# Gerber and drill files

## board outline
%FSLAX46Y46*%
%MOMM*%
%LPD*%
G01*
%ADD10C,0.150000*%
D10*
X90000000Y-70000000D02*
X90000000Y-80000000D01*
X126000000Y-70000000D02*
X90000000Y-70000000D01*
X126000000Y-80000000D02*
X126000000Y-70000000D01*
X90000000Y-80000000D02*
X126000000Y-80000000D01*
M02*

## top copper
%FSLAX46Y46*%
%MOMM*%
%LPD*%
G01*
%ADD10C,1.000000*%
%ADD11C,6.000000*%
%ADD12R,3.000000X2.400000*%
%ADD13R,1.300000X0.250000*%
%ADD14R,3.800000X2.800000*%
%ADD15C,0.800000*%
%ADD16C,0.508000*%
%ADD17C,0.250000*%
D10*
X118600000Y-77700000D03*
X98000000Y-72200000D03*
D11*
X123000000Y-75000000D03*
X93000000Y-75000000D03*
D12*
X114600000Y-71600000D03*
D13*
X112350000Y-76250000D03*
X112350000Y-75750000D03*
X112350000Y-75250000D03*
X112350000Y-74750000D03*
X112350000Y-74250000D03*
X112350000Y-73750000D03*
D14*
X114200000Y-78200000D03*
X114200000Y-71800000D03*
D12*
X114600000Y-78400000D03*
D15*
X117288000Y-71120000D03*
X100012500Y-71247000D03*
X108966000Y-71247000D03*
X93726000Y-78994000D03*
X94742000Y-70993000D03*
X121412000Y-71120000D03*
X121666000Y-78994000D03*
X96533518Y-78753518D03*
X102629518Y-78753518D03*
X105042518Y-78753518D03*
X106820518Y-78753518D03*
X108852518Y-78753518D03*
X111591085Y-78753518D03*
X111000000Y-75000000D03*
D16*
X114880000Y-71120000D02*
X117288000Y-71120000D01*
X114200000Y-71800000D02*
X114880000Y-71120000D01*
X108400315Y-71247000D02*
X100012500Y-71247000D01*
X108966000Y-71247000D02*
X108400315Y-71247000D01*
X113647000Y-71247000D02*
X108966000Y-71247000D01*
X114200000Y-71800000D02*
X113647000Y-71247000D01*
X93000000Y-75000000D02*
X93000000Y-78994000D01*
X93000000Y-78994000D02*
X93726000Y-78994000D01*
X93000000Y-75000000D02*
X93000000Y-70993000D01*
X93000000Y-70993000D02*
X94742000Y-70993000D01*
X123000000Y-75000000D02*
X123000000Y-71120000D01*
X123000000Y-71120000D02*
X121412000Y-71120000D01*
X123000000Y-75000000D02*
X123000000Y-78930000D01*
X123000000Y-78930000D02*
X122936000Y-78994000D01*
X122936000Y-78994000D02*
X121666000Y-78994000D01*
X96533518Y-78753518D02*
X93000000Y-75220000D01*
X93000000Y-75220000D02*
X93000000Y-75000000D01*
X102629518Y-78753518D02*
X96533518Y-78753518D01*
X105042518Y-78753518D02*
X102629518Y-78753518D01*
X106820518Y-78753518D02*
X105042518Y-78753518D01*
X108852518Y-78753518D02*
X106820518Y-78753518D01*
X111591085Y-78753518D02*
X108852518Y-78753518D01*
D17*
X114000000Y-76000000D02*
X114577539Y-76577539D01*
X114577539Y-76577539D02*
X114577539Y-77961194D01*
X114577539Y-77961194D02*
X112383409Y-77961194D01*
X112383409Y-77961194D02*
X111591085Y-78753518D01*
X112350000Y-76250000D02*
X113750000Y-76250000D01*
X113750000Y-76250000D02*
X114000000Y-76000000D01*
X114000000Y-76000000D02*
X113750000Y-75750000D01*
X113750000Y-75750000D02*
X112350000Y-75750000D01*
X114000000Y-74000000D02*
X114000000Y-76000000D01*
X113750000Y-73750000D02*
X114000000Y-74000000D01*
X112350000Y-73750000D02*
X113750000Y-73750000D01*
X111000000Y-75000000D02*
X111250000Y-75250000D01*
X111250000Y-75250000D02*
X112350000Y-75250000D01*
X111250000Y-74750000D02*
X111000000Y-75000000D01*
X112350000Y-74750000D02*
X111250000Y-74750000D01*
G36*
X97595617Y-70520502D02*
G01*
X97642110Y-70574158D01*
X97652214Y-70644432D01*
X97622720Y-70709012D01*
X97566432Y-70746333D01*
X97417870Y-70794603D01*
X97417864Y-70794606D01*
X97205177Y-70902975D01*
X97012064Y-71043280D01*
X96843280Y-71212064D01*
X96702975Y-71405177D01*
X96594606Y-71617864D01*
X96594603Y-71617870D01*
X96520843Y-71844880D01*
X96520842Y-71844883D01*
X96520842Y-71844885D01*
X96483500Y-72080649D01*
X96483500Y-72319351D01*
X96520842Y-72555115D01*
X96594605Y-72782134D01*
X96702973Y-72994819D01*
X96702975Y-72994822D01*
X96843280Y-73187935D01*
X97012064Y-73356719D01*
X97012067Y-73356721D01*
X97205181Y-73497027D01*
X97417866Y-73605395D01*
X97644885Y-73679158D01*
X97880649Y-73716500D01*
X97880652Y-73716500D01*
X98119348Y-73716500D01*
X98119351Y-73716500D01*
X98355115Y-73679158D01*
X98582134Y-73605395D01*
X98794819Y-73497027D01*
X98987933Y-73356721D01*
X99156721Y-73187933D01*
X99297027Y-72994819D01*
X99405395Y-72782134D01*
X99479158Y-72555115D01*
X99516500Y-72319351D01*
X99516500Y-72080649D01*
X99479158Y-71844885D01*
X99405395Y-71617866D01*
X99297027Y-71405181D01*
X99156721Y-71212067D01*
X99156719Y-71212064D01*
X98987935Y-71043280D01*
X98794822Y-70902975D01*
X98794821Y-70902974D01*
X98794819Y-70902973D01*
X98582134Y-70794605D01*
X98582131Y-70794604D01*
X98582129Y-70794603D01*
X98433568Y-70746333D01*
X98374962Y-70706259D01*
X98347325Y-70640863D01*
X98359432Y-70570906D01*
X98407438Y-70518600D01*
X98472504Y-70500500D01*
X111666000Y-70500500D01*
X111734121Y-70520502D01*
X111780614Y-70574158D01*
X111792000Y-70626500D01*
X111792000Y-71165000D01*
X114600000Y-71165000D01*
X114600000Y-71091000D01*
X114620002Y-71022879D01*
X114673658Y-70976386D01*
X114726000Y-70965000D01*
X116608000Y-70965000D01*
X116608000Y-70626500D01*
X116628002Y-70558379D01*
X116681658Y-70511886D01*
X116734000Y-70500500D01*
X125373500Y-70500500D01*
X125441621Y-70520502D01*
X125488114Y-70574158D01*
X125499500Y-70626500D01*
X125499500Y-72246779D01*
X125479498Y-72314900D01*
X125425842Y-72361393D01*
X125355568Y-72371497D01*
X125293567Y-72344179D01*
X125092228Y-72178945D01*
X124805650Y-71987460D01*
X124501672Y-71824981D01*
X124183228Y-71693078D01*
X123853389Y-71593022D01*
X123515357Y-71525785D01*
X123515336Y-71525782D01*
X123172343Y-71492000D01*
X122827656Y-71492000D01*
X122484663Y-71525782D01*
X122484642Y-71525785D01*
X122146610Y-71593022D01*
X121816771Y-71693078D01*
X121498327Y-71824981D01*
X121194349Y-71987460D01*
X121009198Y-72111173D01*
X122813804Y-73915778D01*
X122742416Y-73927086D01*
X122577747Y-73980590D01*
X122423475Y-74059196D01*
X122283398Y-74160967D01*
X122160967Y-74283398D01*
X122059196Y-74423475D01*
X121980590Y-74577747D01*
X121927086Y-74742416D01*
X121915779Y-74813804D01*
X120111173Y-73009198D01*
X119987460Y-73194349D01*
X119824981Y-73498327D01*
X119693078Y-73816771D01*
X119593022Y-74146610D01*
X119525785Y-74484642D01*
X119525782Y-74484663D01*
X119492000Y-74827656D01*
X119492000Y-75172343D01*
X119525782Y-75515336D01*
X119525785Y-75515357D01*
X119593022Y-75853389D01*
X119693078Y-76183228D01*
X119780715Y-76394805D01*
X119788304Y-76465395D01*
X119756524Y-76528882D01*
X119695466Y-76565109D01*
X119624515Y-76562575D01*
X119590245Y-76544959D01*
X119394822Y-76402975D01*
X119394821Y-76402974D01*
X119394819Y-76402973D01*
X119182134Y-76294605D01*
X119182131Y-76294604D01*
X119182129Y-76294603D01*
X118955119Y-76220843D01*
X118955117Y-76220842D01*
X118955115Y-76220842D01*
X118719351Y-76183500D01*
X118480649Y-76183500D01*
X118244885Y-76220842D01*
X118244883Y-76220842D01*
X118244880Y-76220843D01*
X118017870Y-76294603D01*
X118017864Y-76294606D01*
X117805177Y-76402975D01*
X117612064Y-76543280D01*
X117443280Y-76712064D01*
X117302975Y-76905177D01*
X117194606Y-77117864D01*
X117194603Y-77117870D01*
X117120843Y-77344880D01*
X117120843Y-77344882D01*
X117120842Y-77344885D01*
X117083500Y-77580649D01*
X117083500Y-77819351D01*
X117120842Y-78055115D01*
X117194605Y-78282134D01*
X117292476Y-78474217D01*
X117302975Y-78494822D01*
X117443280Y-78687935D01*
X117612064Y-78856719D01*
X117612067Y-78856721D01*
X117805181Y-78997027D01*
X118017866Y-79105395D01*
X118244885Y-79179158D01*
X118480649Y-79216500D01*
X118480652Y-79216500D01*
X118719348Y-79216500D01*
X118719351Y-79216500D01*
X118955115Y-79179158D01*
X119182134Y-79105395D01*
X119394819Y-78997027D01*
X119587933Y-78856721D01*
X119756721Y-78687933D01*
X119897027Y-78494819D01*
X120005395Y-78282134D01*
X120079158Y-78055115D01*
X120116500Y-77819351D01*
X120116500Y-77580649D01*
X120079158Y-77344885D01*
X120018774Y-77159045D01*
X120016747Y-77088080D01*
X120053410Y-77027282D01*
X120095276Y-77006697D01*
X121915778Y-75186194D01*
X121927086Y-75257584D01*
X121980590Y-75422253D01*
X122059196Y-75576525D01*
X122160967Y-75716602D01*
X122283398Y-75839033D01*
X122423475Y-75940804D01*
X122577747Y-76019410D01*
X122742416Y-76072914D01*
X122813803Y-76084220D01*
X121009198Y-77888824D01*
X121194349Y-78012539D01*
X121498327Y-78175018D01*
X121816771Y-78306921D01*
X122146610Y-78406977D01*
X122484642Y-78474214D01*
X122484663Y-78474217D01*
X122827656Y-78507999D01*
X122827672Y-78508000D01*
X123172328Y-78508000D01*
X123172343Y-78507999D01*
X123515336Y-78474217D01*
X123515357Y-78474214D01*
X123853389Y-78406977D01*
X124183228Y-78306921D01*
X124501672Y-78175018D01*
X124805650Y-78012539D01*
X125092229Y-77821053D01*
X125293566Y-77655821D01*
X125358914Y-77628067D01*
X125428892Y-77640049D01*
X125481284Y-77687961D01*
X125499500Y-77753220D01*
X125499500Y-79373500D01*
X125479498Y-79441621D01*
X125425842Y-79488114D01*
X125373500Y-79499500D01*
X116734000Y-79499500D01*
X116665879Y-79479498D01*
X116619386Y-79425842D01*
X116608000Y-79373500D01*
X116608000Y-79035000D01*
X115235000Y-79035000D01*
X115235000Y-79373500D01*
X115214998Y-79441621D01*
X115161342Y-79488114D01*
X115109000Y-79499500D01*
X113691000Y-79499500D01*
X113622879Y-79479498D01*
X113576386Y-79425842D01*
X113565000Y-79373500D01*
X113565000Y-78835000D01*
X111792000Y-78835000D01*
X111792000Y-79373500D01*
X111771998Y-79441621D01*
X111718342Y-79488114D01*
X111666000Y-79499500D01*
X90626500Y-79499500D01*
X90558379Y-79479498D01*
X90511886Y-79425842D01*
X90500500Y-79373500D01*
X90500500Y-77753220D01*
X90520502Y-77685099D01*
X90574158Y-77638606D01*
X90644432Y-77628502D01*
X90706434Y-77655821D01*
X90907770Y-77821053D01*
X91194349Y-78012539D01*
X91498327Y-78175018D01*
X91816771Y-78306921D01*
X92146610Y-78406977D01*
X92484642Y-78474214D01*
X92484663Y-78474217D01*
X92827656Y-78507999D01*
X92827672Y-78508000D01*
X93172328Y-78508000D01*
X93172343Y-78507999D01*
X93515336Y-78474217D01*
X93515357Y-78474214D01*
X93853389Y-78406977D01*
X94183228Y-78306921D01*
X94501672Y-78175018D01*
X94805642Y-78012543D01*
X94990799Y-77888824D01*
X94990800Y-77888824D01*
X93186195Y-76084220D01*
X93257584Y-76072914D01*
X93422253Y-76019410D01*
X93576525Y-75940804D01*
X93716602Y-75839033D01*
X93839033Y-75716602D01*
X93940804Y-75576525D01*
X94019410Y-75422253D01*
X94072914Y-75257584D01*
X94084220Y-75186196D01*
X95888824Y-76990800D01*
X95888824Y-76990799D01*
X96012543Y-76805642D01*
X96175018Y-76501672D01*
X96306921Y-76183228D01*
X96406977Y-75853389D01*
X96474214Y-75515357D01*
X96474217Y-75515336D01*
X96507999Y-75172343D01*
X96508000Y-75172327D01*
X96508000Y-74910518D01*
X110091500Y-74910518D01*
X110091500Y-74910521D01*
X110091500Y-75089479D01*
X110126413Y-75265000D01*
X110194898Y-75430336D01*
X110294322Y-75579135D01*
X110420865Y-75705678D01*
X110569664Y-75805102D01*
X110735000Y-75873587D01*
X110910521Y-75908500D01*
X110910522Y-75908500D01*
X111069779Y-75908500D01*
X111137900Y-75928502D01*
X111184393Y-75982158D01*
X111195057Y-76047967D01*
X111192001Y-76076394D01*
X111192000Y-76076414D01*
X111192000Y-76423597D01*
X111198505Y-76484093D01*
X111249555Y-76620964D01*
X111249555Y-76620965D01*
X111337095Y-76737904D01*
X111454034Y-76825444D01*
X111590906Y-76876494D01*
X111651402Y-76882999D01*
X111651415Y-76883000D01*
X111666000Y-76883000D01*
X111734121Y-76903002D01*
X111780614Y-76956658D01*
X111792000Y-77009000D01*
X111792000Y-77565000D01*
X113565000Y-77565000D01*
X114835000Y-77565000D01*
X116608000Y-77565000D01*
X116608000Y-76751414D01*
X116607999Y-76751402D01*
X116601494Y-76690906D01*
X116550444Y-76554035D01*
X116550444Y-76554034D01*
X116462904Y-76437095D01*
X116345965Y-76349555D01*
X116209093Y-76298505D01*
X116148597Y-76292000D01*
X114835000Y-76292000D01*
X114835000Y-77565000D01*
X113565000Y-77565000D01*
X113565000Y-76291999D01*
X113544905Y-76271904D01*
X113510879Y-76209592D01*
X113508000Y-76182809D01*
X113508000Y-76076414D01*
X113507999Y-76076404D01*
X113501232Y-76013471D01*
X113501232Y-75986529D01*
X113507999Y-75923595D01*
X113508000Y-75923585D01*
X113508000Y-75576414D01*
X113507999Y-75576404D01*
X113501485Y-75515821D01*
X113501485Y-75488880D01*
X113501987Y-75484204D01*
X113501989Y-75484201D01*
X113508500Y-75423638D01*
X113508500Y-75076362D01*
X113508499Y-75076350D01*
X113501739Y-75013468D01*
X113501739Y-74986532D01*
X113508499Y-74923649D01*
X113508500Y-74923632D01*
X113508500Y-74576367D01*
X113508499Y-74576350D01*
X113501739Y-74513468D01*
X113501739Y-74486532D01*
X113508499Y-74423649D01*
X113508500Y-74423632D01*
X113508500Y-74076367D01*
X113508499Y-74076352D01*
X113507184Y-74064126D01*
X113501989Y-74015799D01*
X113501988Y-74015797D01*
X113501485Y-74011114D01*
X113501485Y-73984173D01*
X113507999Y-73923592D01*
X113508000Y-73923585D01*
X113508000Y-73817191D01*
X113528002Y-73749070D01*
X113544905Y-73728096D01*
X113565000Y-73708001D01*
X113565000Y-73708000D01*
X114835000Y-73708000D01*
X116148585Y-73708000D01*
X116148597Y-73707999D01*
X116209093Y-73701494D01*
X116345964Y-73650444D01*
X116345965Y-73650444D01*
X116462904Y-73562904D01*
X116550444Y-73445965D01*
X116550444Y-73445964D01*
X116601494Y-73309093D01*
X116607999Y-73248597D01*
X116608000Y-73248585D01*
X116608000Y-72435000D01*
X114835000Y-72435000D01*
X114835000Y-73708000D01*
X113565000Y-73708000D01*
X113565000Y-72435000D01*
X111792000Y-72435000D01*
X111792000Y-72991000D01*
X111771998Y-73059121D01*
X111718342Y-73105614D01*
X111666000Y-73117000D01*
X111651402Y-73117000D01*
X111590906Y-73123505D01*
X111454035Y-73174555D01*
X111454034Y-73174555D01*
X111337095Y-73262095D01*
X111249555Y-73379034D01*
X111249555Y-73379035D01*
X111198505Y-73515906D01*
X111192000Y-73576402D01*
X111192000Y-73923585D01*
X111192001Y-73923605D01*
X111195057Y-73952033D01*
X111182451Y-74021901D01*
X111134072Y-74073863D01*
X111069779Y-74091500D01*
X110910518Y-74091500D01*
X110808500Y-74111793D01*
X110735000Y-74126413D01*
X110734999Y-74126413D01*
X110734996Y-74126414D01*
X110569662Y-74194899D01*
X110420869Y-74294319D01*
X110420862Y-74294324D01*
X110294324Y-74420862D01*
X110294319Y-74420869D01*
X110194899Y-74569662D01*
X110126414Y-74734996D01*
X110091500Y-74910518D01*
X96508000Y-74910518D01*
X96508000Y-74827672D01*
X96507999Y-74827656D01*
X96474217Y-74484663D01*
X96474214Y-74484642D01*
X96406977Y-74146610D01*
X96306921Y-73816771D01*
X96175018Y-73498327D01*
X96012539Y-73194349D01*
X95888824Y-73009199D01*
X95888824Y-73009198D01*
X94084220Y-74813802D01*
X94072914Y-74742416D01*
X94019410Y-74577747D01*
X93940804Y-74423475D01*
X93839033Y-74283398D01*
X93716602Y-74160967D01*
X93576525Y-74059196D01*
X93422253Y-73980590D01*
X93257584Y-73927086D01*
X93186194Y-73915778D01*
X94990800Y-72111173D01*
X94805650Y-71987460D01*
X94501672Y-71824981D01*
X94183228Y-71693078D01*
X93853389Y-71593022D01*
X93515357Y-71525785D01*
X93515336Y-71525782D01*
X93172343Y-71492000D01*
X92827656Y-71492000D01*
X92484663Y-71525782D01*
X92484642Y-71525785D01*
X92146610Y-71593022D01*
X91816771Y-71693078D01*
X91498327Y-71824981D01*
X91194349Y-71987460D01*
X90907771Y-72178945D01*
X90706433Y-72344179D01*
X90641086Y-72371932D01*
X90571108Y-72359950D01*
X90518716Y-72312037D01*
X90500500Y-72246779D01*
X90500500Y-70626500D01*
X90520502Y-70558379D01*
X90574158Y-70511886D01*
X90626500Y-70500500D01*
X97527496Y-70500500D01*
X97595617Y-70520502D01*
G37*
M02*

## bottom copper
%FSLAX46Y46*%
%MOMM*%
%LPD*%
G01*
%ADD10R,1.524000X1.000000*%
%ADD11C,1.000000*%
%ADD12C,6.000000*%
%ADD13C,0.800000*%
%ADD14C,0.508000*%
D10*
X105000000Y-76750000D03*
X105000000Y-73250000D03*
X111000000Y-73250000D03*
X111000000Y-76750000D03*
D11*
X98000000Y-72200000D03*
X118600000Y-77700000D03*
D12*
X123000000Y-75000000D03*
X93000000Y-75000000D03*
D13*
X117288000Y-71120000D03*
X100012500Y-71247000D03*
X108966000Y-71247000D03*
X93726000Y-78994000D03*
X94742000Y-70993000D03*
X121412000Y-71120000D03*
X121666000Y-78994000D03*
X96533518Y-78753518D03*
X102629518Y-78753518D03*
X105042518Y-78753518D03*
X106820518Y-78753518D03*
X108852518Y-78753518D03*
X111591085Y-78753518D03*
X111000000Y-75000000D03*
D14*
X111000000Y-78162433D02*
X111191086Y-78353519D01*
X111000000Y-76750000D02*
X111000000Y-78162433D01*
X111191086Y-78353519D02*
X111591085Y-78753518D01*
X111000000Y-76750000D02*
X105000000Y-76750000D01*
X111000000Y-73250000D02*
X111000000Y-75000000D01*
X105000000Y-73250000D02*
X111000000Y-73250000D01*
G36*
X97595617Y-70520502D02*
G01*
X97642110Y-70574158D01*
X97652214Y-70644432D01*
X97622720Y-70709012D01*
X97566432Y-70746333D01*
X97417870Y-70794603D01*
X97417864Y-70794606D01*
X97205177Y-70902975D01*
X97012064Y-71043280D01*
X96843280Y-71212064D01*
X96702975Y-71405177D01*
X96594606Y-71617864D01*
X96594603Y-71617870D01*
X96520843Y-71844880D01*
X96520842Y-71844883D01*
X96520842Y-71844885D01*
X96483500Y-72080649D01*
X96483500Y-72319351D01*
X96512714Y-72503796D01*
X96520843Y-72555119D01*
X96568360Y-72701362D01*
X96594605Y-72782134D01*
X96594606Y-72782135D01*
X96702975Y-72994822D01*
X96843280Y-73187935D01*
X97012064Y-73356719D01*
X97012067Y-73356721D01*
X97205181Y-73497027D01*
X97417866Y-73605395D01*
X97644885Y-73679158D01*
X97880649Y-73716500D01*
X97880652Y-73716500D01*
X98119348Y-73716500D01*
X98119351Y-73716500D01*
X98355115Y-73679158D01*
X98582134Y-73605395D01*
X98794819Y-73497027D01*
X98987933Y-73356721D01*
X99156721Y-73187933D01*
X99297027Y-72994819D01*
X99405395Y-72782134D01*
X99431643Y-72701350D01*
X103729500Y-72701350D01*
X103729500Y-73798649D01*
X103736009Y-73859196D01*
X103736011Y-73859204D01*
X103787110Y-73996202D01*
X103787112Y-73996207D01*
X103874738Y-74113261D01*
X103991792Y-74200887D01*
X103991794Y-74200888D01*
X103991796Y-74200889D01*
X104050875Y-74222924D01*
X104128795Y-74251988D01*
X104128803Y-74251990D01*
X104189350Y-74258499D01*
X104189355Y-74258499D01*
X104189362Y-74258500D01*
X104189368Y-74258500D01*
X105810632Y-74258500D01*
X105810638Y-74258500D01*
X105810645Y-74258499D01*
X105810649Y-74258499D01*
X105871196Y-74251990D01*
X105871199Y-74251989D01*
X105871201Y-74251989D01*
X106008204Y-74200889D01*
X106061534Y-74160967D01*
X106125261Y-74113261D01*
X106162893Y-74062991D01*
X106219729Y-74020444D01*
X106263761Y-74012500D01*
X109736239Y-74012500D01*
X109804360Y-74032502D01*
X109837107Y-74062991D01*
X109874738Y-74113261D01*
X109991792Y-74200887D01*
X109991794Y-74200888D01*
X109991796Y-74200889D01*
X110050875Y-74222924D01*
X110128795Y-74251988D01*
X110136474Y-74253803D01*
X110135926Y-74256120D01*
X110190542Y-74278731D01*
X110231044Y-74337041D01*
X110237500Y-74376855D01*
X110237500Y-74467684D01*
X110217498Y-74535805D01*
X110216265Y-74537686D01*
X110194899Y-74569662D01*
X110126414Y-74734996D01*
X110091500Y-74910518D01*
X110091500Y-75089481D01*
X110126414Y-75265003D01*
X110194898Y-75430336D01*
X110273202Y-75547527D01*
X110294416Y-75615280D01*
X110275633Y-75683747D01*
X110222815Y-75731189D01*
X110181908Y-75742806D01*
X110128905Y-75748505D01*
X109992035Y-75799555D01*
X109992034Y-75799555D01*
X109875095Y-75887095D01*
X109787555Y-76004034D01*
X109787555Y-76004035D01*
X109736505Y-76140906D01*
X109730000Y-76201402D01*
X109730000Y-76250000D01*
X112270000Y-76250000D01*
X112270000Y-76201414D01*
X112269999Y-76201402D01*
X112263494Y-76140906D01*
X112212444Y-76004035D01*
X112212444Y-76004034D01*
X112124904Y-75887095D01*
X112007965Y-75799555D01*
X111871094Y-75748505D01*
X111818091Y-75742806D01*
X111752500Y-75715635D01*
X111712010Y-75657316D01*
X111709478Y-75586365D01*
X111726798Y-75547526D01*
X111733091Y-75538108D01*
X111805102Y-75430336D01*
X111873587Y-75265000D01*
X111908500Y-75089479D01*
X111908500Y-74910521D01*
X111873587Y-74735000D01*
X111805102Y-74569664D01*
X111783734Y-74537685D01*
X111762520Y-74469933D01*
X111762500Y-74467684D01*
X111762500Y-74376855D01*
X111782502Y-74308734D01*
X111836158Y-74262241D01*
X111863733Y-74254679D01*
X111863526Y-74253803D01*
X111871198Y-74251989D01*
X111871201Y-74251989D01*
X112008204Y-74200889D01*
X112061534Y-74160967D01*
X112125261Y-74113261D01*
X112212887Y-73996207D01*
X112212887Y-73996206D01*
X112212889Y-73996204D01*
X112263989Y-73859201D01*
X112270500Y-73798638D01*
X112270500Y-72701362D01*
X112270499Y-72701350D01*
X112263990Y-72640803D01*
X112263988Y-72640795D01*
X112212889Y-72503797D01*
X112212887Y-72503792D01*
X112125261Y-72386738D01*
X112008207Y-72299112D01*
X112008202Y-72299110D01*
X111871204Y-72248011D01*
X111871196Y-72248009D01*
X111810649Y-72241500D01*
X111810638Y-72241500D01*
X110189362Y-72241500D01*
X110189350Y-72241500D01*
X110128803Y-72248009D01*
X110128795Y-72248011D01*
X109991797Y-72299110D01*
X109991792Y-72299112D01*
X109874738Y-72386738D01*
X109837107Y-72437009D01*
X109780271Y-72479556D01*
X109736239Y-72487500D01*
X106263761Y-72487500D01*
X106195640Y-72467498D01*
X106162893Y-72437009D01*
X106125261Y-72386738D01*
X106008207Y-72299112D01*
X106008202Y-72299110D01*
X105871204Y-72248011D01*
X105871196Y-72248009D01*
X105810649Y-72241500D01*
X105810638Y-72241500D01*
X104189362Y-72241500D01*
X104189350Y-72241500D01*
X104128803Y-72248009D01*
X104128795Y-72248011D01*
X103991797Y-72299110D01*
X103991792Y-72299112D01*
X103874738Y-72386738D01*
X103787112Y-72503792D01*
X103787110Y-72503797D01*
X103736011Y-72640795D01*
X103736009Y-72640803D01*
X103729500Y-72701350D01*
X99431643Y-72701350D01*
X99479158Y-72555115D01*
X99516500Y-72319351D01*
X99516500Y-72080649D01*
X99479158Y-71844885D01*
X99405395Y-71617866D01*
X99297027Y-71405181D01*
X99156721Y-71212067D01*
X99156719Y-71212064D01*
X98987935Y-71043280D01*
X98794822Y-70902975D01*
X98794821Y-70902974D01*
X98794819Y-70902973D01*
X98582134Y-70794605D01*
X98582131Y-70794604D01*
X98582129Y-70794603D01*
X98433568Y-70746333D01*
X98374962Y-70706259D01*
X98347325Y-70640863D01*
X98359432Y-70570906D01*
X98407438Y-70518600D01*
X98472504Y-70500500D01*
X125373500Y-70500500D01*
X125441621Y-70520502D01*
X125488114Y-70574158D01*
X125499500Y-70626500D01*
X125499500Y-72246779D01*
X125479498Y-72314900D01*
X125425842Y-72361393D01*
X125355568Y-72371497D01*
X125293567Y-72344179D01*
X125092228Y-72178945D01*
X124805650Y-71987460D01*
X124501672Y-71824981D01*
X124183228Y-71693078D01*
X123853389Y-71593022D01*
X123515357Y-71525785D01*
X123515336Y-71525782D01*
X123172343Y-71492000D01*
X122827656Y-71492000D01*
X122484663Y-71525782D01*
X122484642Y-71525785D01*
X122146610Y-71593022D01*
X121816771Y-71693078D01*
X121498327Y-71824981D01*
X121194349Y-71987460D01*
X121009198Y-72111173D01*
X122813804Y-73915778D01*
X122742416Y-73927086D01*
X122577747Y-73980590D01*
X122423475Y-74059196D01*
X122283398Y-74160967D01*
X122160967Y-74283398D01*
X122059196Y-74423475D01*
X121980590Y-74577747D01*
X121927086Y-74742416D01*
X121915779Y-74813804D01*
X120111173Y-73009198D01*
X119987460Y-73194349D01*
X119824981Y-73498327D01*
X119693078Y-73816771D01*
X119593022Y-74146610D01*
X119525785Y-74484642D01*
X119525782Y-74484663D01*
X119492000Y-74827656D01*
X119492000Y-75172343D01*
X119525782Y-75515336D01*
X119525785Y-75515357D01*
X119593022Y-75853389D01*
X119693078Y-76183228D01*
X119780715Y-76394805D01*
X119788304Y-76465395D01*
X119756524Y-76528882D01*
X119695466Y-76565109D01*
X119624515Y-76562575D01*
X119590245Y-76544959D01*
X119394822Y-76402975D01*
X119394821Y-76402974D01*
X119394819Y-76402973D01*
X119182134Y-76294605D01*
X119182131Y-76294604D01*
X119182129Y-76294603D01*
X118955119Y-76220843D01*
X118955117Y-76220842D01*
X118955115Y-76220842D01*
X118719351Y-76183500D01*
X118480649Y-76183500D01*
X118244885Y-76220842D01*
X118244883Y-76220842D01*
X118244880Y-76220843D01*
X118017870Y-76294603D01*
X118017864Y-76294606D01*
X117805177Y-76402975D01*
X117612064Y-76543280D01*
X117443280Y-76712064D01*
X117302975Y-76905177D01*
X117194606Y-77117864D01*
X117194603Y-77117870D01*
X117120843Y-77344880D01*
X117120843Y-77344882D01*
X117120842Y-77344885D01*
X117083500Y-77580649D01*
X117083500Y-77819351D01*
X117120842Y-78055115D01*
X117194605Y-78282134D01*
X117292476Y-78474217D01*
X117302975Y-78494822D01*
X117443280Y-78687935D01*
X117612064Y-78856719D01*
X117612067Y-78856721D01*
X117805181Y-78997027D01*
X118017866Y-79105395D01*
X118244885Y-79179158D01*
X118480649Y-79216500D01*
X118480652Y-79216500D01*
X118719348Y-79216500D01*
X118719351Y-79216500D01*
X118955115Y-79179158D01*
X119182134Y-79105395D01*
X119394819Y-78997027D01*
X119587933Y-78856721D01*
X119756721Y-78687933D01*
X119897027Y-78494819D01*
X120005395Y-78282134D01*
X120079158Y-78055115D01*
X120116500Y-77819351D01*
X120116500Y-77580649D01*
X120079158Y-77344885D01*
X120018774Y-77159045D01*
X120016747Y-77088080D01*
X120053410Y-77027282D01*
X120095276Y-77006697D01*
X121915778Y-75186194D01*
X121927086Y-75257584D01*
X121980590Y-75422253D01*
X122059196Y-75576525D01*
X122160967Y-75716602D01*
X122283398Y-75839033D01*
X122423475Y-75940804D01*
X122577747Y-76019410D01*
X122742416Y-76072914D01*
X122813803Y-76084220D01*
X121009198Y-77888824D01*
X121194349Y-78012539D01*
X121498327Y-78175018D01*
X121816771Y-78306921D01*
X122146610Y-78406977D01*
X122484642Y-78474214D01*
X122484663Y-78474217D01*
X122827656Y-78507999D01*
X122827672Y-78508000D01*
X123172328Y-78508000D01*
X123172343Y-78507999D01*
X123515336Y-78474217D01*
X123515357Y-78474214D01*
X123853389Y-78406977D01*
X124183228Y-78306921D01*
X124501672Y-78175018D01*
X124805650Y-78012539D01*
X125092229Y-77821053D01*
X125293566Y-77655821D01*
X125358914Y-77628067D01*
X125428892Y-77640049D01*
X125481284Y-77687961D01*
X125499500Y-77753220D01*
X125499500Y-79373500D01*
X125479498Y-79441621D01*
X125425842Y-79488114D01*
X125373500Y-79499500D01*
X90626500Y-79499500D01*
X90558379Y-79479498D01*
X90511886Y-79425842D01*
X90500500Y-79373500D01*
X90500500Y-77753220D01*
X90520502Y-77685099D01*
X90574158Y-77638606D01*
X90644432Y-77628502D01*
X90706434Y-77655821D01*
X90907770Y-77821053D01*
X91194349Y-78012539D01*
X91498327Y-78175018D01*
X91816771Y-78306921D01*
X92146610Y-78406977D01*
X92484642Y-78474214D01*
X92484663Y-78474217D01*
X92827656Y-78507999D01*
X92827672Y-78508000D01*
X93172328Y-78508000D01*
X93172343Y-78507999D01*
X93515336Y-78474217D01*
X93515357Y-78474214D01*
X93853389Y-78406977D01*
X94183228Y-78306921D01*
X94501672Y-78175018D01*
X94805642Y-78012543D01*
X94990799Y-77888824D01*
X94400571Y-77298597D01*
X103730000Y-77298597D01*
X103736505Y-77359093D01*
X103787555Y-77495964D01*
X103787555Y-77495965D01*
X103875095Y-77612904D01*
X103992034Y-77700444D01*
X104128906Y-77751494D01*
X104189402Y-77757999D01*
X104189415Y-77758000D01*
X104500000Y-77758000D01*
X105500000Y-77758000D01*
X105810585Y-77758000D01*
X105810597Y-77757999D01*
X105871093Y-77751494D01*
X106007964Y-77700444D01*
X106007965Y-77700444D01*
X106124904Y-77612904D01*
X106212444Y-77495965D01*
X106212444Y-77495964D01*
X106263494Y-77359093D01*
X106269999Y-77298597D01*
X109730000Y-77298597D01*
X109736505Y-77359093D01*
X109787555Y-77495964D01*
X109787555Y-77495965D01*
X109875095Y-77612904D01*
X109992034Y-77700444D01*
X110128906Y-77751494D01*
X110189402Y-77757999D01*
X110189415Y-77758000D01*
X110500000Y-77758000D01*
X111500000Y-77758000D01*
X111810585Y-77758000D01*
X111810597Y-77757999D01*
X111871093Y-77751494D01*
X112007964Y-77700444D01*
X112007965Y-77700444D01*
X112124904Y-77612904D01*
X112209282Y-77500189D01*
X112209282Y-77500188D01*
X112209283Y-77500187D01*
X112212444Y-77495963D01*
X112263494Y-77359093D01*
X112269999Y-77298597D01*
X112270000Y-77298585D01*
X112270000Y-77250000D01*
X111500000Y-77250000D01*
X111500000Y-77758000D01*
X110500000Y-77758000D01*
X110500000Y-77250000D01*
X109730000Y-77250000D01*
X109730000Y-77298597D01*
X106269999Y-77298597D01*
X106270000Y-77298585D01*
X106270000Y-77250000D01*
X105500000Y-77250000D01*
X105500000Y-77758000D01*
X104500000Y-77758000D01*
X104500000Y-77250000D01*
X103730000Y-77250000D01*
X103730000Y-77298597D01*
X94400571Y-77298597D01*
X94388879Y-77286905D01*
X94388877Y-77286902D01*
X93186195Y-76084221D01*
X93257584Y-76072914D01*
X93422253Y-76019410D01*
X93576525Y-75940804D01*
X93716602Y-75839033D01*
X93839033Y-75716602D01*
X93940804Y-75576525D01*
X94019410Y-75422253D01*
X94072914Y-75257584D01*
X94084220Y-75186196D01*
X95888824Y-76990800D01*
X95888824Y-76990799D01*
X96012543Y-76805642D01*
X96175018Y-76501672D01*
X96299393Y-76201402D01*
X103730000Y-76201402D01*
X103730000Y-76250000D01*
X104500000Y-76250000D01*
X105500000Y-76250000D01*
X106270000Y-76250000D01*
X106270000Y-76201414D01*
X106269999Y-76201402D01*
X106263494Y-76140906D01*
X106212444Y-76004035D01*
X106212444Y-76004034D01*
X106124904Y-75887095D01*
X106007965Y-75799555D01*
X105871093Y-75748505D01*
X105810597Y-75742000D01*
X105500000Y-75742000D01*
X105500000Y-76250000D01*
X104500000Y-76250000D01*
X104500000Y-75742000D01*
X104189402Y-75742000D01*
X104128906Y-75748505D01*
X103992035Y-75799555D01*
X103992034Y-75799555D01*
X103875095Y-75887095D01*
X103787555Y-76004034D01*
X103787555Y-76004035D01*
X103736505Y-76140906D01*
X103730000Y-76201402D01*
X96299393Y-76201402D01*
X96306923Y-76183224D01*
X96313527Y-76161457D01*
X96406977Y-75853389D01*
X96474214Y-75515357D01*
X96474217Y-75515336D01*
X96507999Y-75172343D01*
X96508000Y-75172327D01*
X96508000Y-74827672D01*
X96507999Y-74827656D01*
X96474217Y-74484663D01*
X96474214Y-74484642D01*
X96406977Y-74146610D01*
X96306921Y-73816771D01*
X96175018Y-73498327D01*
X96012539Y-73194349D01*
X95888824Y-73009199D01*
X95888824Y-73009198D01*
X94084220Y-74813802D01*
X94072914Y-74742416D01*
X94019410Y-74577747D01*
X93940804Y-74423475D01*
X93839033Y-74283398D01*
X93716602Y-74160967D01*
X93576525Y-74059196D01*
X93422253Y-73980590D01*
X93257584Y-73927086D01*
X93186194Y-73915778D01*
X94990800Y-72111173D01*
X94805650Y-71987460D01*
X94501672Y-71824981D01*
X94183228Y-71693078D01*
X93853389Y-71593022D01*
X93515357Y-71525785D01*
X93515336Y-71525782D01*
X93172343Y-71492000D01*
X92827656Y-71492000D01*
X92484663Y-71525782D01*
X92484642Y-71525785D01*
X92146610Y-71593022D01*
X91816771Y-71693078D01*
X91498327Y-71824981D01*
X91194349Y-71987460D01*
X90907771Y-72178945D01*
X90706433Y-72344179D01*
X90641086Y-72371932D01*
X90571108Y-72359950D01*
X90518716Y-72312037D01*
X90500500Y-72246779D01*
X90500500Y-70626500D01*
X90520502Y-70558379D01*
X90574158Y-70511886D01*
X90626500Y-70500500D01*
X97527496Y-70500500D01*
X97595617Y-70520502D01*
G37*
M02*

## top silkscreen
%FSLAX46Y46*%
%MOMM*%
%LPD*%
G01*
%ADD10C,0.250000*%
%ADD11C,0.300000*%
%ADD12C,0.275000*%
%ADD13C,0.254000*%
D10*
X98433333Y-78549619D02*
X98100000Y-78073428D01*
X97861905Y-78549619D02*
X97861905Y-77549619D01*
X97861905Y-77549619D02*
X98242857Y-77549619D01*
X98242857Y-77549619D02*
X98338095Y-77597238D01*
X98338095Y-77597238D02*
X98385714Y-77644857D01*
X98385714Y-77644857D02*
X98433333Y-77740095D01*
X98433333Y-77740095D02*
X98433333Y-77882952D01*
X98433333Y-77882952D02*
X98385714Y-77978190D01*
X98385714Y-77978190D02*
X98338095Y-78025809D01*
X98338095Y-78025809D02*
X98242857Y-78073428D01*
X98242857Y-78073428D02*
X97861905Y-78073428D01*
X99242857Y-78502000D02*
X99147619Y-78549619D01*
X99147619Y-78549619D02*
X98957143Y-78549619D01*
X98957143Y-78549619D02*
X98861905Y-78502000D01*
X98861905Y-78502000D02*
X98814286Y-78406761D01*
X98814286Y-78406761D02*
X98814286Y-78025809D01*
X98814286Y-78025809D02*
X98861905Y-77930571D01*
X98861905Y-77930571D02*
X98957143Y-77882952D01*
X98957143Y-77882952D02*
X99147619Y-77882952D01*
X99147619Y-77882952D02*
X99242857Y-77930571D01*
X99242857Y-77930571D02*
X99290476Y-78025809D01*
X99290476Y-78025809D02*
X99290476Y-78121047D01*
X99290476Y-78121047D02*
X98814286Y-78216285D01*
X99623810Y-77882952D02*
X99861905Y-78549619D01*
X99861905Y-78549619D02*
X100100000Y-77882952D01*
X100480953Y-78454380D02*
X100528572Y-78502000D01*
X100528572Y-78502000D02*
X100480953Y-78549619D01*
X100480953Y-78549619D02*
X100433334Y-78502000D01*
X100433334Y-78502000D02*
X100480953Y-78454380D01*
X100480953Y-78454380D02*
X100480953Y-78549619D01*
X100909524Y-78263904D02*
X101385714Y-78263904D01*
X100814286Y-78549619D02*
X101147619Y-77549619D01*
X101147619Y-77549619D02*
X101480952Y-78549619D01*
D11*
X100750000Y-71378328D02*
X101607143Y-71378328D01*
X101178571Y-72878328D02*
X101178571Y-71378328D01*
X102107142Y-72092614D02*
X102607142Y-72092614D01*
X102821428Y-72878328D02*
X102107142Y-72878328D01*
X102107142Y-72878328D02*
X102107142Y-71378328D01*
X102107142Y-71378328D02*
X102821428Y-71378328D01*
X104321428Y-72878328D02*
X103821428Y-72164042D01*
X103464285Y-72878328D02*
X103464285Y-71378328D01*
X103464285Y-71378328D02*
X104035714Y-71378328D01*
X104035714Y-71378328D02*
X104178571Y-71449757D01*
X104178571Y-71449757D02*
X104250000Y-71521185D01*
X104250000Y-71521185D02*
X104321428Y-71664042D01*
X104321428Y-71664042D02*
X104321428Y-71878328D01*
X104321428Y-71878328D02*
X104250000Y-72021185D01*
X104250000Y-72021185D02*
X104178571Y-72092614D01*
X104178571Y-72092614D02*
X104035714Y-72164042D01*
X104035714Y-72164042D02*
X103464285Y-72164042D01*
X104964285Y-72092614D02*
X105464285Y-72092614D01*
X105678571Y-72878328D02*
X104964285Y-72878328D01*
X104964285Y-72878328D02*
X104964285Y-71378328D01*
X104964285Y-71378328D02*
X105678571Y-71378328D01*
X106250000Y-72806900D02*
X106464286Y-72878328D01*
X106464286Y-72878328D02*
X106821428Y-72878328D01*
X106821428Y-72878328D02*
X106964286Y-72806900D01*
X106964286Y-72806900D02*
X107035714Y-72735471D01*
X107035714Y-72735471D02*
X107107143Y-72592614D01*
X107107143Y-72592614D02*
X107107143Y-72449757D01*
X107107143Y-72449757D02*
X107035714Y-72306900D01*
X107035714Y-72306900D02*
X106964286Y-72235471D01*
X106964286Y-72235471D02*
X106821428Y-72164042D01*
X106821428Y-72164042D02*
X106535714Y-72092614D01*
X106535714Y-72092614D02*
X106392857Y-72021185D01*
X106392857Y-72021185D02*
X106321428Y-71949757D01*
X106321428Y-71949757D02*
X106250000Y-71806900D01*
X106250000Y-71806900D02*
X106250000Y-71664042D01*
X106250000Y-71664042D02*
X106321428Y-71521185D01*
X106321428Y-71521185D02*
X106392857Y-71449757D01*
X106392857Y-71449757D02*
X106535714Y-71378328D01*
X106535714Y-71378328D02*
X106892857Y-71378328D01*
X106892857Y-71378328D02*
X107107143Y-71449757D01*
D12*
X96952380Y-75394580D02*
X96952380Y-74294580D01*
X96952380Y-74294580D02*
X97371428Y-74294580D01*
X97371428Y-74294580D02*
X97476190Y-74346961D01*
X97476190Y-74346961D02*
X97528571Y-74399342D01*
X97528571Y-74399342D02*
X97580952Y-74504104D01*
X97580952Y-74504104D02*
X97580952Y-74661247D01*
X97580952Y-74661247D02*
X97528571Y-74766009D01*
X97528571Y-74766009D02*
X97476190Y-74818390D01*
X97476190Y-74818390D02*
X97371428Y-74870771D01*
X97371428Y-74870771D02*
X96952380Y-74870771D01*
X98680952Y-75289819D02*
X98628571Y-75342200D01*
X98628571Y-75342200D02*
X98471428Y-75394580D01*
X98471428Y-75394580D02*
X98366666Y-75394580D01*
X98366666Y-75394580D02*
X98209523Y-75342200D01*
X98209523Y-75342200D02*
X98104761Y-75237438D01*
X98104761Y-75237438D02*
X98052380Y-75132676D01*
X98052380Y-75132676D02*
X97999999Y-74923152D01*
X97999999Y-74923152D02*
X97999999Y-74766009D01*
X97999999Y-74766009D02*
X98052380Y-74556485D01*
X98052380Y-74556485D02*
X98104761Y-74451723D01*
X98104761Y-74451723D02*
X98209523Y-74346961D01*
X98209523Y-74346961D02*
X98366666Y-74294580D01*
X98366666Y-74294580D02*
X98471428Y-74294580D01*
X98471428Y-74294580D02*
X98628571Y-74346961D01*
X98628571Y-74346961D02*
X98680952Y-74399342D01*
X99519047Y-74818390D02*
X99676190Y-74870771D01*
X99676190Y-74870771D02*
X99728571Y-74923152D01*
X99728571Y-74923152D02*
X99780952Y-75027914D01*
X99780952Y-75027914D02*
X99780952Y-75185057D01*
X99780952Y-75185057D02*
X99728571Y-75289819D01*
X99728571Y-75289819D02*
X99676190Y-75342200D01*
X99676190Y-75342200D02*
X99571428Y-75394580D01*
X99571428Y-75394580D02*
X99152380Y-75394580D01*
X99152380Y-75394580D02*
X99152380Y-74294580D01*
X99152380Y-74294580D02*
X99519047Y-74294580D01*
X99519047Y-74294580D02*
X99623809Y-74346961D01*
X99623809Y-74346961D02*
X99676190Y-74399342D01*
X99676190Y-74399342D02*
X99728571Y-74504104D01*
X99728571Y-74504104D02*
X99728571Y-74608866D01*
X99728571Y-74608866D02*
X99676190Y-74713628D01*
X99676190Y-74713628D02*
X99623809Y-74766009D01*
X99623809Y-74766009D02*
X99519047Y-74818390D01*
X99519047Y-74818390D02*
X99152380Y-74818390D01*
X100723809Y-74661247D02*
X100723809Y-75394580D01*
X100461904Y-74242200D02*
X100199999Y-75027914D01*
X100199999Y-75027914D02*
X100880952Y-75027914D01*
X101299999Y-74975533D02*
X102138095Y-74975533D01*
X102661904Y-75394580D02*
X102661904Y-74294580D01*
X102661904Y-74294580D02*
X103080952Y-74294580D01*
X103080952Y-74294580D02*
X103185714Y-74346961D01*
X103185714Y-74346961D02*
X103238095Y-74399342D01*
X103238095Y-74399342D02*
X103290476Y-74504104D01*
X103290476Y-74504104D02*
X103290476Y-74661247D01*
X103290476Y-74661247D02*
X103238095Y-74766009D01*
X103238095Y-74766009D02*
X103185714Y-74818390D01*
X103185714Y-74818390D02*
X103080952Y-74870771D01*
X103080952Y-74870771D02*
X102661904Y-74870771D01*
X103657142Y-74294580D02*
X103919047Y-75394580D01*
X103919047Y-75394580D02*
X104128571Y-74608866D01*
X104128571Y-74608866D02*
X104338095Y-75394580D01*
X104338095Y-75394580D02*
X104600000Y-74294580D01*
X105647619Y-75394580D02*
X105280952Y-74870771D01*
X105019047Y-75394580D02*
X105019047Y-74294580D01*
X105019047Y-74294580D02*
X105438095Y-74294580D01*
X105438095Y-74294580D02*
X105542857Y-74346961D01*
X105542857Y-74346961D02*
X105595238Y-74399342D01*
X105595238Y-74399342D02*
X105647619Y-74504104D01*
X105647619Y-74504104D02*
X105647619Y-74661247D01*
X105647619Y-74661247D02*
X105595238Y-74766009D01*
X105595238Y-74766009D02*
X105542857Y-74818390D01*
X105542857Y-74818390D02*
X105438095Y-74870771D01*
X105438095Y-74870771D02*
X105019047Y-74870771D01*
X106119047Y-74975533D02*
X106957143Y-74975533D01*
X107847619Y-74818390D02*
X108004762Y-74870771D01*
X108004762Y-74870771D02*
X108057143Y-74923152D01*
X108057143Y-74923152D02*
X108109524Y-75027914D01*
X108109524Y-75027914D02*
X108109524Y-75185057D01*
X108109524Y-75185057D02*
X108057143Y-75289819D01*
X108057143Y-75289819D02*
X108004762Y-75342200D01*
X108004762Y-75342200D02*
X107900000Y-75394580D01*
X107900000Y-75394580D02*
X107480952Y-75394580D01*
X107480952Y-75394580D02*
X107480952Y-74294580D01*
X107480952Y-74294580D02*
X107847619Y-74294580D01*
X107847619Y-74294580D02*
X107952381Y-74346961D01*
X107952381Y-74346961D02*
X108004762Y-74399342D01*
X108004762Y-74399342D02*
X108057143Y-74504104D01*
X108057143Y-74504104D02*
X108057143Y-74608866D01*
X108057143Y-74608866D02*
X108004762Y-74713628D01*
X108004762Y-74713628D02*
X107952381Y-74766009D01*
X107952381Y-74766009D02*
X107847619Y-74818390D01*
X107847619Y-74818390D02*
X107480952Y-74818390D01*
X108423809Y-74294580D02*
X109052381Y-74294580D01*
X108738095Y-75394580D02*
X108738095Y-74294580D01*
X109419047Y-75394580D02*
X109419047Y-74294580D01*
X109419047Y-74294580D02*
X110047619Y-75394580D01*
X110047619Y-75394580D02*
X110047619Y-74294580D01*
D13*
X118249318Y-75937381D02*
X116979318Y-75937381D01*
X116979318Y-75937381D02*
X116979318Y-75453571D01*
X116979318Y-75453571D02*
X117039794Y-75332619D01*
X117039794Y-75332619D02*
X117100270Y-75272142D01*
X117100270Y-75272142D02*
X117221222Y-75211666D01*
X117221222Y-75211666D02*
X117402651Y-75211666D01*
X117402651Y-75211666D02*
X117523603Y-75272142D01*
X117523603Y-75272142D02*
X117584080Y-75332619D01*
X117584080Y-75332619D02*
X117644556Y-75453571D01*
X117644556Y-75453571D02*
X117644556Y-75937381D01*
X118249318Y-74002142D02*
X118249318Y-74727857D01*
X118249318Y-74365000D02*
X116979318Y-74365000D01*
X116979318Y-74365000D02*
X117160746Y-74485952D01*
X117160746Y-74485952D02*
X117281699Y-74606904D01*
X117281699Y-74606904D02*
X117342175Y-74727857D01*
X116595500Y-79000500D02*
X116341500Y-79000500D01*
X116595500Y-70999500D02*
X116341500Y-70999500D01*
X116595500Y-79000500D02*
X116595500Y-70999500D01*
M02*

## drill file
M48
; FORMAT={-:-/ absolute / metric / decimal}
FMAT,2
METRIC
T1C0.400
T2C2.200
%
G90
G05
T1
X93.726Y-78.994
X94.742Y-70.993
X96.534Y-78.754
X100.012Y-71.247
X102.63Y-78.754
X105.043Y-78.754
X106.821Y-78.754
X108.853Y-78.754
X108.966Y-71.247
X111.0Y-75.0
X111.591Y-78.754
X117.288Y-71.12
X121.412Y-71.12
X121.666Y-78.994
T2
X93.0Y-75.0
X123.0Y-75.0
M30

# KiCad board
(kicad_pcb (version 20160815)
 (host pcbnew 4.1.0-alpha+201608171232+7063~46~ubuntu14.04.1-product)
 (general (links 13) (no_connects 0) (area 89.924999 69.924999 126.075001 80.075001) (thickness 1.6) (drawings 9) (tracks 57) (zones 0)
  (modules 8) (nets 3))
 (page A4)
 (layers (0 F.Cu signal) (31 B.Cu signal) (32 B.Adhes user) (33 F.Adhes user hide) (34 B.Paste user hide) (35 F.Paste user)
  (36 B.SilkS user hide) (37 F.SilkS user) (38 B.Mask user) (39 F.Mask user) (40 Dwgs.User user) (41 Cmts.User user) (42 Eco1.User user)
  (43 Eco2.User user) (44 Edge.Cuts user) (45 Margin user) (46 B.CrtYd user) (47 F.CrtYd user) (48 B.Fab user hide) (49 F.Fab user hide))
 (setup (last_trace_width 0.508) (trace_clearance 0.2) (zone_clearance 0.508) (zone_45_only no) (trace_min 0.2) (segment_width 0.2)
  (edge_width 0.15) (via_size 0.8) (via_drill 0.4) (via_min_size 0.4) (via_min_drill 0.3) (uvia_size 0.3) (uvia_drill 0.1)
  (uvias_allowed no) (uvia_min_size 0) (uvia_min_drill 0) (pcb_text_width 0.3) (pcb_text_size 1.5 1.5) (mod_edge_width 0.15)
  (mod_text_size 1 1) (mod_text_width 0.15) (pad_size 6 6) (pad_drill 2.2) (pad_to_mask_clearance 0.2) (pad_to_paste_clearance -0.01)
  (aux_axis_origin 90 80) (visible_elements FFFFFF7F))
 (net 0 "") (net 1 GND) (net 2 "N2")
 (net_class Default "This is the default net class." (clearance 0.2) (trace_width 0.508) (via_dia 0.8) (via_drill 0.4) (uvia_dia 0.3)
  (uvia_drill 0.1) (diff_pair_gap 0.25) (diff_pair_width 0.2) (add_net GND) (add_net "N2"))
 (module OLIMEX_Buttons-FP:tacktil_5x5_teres (layer B.Cu) (at 108 75)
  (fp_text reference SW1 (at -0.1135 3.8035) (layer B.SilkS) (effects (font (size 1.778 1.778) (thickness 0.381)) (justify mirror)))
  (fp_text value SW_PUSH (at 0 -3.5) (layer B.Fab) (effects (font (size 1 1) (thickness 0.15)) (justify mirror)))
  (pad 1 smd rect (at -3 1.75) (size 1.524 1) (layers B.Cu B.Paste B.Mask) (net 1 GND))
  (pad 2 smd rect (at -3 -1.75) (size 1.524 1) (layers B.Cu B.Paste B.Mask) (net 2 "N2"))
  (pad 2 smd rect (at 3 -1.75) (size 1.524 1) (layers B.Cu B.Paste B.Mask) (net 2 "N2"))
  (pad 1 smd rect (at 3 1.75) (size 1.524 1) (layers B.Cu B.Paste B.Mask) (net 1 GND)))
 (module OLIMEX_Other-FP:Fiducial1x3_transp (layer B.Cu) (at 98 72.2)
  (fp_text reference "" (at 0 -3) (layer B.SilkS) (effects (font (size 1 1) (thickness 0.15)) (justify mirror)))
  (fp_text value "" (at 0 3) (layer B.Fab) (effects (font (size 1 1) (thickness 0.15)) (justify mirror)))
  (pad Fid1 connect circle (at 0 0) (size 1 1) (layers B.Cu B.Mask) (solder_mask_margin 0.127) (clearance 1.016) (zone_connect 0)))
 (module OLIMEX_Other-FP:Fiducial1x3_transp (layer B.Cu) (at 118.6 77.7)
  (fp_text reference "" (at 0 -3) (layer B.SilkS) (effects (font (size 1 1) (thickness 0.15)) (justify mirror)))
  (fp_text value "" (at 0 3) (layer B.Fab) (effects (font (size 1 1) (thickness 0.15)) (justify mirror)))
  (pad Fid1 connect circle (at 0 0) (size 1 1) (layers B.Cu B.Mask) (solder_mask_margin 0.127) (clearance 1.016) (zone_connect 0)))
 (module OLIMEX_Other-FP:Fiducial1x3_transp (layer F.Cu) (at 118.6 77.7)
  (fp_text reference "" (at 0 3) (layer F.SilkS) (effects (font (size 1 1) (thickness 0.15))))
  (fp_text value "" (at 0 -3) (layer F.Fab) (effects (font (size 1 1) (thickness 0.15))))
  (pad Fid1 connect circle (at 0 0) (size 1 1) (layers F.Cu F.Mask) (solder_mask_margin 0.127) (clearance 1.016) (zone_connect 0)))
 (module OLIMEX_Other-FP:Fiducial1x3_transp (layer F.Cu) (at 98 72.2)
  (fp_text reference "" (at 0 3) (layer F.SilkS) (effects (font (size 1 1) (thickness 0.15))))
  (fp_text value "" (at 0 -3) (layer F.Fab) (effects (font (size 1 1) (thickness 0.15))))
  (pad Fid1 connect circle (at 0 0) (size 1 1) (layers F.Cu F.Mask) (solder_mask_margin 0.127) (clearance 1.016) (zone_connect 0)))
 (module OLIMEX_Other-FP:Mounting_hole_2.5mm (layer F.Cu) (at 123 75)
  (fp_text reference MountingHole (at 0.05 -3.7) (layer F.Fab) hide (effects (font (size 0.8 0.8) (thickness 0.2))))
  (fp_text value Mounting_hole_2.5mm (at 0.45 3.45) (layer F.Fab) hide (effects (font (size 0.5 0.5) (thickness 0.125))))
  (pad "" thru_hole circle (at 0 0) (size 6 6) (drill 2.2) (layers *.Cu *.Mask) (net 1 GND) (clearance 1.55)))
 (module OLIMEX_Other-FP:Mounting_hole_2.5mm (layer F.Cu) (at 93 75)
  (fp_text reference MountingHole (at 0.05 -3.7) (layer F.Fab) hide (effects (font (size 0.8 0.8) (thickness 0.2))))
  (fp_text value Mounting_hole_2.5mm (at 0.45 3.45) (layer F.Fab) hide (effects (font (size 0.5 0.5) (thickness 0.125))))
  (pad "" thru_hole circle (at 0 0) (size 6 6) (drill 2.2) (layers *.Cu *.Mask) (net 1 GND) (clearance 1.55)))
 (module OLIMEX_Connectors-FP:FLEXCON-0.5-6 (layer F.Cu) (at 114.5 75 90)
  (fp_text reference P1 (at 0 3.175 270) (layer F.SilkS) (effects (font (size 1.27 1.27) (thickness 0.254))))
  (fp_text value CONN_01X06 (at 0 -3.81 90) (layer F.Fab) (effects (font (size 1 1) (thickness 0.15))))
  (fp_line (start -4.0005 2.0955) (end -4.0005 1.8415) (layer F.SilkS) (width 0.254))
  (fp_line (start 4.0005 2.0955) (end 4.0005 1.8415) (layer F.SilkS) (width 0.254))
  (fp_line (start -4.0005 2.0955) (end 4.0005 2.0955) (layer F.SilkS) (width 0.254))
  (pad 0 smd rect (at 3.4 0.1 90) (size 2.4 3) (layers F.Cu F.Paste F.Mask) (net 1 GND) (solder_mask_margin -0.01)
   (solder_paste_margin -0.01))
  (pad 1 smd rect (at -1.25 -2.15 90) (size 0.25 1.3) (layers F.Cu F.Paste F.Mask) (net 1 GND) (solder_mask_margin 0.0508)
   (solder_paste_margin -0.01))
  (pad 2 smd rect (at -0.75 -2.15 90) (size 0.25 1.3) (layers F.Cu F.Paste F.Mask) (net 1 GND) (solder_mask_margin 0.0508)
   (solder_paste_margin -0.01))
  (pad 3 smd rect (at -0.25 -2.15 90) (size 0.25 1.3) (layers F.Cu F.Paste F.Mask) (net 2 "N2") (solder_mask_margin 0.0508)
   (solder_paste_margin -0.01))
  (pad 4 smd rect (at 0.25 -2.15 90) (size 0.25 1.3) (layers F.Cu F.Paste F.Mask) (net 2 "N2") (solder_mask_margin 0.0508)
   (solder_paste_margin -0.01))
  (pad 5 smd rect (at 0.75 -2.15 90) (size 0.25 1.3) (layers F.Cu F.Paste F.Mask) (solder_mask_margin 0.0508) (solder_paste_margin -0.01))
  (pad 6 smd rect (at 1.25 -2.15 90) (size 0.25 1.3) (layers F.Cu F.Paste F.Mask) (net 1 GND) (solder_mask_margin 0.0508)
   (solder_paste_margin -0.01))
  (pad 0 smd rect (at -3.2 -0.3 90) (size 2.8 3.8) (layers F.Cu) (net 1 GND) (solder_mask_margin -0.1) (solder_paste_margin -0.1))
  (pad 0 smd rect (at 3.2 -0.3 90) (size 2.8 3.8) (layers F.Cu) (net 1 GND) (solder_mask_margin -0.1) (solder_paste_margin -0.1))
  (pad 0 smd rect (at -3.4 0.1 90) (size 2.4 3) (layers F.Cu F.Paste F.Mask) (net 1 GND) (solder_mask_margin -0.01)
   (solder_paste_margin -0.01)))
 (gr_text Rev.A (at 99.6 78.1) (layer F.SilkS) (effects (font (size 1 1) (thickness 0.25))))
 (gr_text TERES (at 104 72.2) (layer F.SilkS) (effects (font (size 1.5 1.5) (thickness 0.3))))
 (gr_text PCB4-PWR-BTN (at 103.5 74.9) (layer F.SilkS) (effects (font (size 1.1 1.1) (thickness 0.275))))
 (gr_line (start 90 70) (end 90 80) (layer Edge.Cuts) (width 0.15))
 (gr_line (start 126 70) (end 90 70) (layer Edge.Cuts) (width 0.15))
 (gr_line (start 126 80) (end 126 70) (layer Edge.Cuts) (width 0.15))
 (gr_line (start 90 80) (end 126 80) (layer Edge.Cuts) (width 0.15))
 (via (at 117.288 71.12) (size 0.8) (drill 0.4) (layers F.Cu B.Cu) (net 1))
 (segment (start 114.88 71.12) (end 117.288 71.12) (width 0.508) (layer F.Cu) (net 1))
 (segment (start 114.2 71.8) (end 114.88 71.12) (width 0.508) (layer F.Cu) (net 1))
 (via (at 100.0125 71.247) (size 0.8) (drill 0.4) (layers F.Cu B.Cu) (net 1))
 (segment (start 108.400315 71.247) (end 100.0125 71.247) (width 0.508) (layer F.Cu) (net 1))
 (segment (start 108.966 71.247) (end 108.400315 71.247) (width 0.508) (layer F.Cu) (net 1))
 (via (at 108.966 71.247) (size 0.8) (drill 0.4) (layers F.Cu B.Cu) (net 1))
 (segment (start 113.647 71.247) (end 108.966 71.247) (width 0.508) (layer F.Cu) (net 1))
 (segment (start 114.2 71.8) (end 113.647 71.247) (width 0.508) (layer F.Cu) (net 1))
 (segment (start 93 75) (end 93 78.994) (width 0.508) (layer F.Cu) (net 1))
 (segment (start 93 78.994) (end 93.726 78.994) (width 0.508) (layer F.Cu) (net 1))
 (via (at 93.726 78.994) (size 0.8) (drill 0.4) (layers F.Cu B.Cu) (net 1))
 (segment (start 93 75) (end 93 70.993) (width 0.508) (layer F.Cu) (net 1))
 (segment (start 93 70.993) (end 94.742 70.993) (width 0.508) (layer F.Cu) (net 1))
 (via (at 94.742 70.993) (size 0.8) (drill 0.4) (layers F.Cu B.Cu) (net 1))
 (segment (start 123 75) (end 123 71.12) (width 0.508) (layer F.Cu) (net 1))
 (segment (start 123 71.12) (end 121.412 71.12) (width 0.508) (layer F.Cu) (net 1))
 (segment (start 123 75) (end 123 78.93) (width 0.508) (layer F.Cu) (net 1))
 (segment (start 123 78.93) (end 122.936 78.994) (width 0.508) (layer F.Cu) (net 1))
 (segment (start 122.936 78.994) (end 121.666 78.994) (width 0.508) (layer F.Cu) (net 1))
 (via (at 121.412 71.12) (size 0.8) (drill 0.4) (layers F.Cu B.Cu) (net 1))
 (via (at 121.666 78.994) (size 0.8) (drill 0.4) (layers F.Cu B.Cu) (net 1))
 (segment (start 96.533518 78.753518) (end 93 75.22) (width 0.508) (layer F.Cu) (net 1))
 (segment (start 93 75.22) (end 93 75) (width 0.508) (layer F.Cu) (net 1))
 (via (at 96.533518 78.753518) (size 0.8) (drill 0.4) (layers F.Cu B.Cu) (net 1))
 (segment (start 102.629518 78.753518) (end 96.533518 78.753518) (width 0.508) (layer F.Cu) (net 1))
 (via (at 102.629518 78.753518) (size 0.8) (drill 0.4) (layers F.Cu B.Cu) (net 1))
 (segment (start 105.042518 78.753518) (end 102.629518 78.753518) (width 0.508) (layer F.Cu) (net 1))
 (via (at 105.042518 78.753518) (size 0.8) (drill 0.4) (layers F.Cu B.Cu) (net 1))
 (segment (start 106.820518 78.753518) (end 105.042518 78.753518) (width 0.508) (layer F.Cu) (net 1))
 (via (at 106.820518 78.753518) (size 0.8) (drill 0.4) (layers F.Cu B.Cu) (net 1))
 (segment (start 108.852518 78.753518) (end 106.820518 78.753518) (width 0.508) (layer F.Cu) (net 1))
 (via (at 108.852518 78.753518) (size 0.8) (drill 0.4) (layers F.Cu B.Cu) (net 1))
 (segment (start 111.591085 78.753518) (end 108.852518 78.753518) (width 0.508) (layer F.Cu) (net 1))
 (segment (start 114 76) (end 114.577539 76.577539) (width 0.25) (layer F.Cu) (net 1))
 (segment (start 114.577539 76.577539) (end 114.577539 77.961194) (width 0.25) (layer F.Cu) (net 1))
 (segment (start 114.577539 77.961194) (end 112.383409 77.961194) (width 0.25) (layer F.Cu) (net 1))
 (segment (start 112.383409 77.961194) (end 111.591085 78.753518) (width 0.25) (layer F.Cu) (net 1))
 (segment (start 111 78.162433) (end 111.191086 78.353519) (width 0.508) (layer B.Cu) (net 1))
 (segment (start 111 76.75) (end 111 78.162433) (width 0.508) (layer B.Cu) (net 1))
 (segment (start 111.191086 78.353519) (end 111.591085 78.753518) (width 0.508) (layer B.Cu) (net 1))
 (via (at 111.591085 78.753518) (size 0.8) (drill 0.4) (layers F.Cu B.Cu) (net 1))
 (segment (start 111 76.75) (end 105 76.75) (width 0.508) (layer B.Cu) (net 1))
 (segment (start 112.35 76.25) (end 113.75 76.25) (width 0.25) (layer F.Cu) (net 1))
 (segment (start 113.75 76.25) (end 114 76) (width 0.25) (layer F.Cu) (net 1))
 (segment (start 114 76) (end 113.75 75.75) (width 0.25) (layer F.Cu) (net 1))
 (segment (start 113.75 75.75) (end 112.35 75.75) (width 0.25) (layer F.Cu) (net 1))
 (segment (start 114 74) (end 114 76) (width 0.25) (layer F.Cu) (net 1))
 (segment (start 113.75 73.75) (end 114 74) (width 0.25) (layer F.Cu) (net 1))
 (segment (start 112.35 73.75) (end 113.75 73.75) (width 0.25) (layer F.Cu) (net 1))
 (segment (start 111 73.25) (end 111 75) (width 0.508) (layer B.Cu) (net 2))
 (segment (start 105 73.25) (end 111 73.25) (width 0.508) (layer B.Cu) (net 2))
 (via (at 111 75) (size 0.8) (drill 0.4) (layers F.Cu B.Cu) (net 2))
 (segment (start 111 75) (end 111.25 75.25) (width 0.25) (layer F.Cu) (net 2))
 (segment (start 111.25 75.25) (end 112.35 75.25) (width 0.25) (layer F.Cu) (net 2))
 (segment (start 111.25 74.75) (end 111 75) (width 0.25) (layer F.Cu) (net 2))
 (segment (start 112.35 74.75) (end 111.25 74.75) (width 0.25) (layer F.Cu) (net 2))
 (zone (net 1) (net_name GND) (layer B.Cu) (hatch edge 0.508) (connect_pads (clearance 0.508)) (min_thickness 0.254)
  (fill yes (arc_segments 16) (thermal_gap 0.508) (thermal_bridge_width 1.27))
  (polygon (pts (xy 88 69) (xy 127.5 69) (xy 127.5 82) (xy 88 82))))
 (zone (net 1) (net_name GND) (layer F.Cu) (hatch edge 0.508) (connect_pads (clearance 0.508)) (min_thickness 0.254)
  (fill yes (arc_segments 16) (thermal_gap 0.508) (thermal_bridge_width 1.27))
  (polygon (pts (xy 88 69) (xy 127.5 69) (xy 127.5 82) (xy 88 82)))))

